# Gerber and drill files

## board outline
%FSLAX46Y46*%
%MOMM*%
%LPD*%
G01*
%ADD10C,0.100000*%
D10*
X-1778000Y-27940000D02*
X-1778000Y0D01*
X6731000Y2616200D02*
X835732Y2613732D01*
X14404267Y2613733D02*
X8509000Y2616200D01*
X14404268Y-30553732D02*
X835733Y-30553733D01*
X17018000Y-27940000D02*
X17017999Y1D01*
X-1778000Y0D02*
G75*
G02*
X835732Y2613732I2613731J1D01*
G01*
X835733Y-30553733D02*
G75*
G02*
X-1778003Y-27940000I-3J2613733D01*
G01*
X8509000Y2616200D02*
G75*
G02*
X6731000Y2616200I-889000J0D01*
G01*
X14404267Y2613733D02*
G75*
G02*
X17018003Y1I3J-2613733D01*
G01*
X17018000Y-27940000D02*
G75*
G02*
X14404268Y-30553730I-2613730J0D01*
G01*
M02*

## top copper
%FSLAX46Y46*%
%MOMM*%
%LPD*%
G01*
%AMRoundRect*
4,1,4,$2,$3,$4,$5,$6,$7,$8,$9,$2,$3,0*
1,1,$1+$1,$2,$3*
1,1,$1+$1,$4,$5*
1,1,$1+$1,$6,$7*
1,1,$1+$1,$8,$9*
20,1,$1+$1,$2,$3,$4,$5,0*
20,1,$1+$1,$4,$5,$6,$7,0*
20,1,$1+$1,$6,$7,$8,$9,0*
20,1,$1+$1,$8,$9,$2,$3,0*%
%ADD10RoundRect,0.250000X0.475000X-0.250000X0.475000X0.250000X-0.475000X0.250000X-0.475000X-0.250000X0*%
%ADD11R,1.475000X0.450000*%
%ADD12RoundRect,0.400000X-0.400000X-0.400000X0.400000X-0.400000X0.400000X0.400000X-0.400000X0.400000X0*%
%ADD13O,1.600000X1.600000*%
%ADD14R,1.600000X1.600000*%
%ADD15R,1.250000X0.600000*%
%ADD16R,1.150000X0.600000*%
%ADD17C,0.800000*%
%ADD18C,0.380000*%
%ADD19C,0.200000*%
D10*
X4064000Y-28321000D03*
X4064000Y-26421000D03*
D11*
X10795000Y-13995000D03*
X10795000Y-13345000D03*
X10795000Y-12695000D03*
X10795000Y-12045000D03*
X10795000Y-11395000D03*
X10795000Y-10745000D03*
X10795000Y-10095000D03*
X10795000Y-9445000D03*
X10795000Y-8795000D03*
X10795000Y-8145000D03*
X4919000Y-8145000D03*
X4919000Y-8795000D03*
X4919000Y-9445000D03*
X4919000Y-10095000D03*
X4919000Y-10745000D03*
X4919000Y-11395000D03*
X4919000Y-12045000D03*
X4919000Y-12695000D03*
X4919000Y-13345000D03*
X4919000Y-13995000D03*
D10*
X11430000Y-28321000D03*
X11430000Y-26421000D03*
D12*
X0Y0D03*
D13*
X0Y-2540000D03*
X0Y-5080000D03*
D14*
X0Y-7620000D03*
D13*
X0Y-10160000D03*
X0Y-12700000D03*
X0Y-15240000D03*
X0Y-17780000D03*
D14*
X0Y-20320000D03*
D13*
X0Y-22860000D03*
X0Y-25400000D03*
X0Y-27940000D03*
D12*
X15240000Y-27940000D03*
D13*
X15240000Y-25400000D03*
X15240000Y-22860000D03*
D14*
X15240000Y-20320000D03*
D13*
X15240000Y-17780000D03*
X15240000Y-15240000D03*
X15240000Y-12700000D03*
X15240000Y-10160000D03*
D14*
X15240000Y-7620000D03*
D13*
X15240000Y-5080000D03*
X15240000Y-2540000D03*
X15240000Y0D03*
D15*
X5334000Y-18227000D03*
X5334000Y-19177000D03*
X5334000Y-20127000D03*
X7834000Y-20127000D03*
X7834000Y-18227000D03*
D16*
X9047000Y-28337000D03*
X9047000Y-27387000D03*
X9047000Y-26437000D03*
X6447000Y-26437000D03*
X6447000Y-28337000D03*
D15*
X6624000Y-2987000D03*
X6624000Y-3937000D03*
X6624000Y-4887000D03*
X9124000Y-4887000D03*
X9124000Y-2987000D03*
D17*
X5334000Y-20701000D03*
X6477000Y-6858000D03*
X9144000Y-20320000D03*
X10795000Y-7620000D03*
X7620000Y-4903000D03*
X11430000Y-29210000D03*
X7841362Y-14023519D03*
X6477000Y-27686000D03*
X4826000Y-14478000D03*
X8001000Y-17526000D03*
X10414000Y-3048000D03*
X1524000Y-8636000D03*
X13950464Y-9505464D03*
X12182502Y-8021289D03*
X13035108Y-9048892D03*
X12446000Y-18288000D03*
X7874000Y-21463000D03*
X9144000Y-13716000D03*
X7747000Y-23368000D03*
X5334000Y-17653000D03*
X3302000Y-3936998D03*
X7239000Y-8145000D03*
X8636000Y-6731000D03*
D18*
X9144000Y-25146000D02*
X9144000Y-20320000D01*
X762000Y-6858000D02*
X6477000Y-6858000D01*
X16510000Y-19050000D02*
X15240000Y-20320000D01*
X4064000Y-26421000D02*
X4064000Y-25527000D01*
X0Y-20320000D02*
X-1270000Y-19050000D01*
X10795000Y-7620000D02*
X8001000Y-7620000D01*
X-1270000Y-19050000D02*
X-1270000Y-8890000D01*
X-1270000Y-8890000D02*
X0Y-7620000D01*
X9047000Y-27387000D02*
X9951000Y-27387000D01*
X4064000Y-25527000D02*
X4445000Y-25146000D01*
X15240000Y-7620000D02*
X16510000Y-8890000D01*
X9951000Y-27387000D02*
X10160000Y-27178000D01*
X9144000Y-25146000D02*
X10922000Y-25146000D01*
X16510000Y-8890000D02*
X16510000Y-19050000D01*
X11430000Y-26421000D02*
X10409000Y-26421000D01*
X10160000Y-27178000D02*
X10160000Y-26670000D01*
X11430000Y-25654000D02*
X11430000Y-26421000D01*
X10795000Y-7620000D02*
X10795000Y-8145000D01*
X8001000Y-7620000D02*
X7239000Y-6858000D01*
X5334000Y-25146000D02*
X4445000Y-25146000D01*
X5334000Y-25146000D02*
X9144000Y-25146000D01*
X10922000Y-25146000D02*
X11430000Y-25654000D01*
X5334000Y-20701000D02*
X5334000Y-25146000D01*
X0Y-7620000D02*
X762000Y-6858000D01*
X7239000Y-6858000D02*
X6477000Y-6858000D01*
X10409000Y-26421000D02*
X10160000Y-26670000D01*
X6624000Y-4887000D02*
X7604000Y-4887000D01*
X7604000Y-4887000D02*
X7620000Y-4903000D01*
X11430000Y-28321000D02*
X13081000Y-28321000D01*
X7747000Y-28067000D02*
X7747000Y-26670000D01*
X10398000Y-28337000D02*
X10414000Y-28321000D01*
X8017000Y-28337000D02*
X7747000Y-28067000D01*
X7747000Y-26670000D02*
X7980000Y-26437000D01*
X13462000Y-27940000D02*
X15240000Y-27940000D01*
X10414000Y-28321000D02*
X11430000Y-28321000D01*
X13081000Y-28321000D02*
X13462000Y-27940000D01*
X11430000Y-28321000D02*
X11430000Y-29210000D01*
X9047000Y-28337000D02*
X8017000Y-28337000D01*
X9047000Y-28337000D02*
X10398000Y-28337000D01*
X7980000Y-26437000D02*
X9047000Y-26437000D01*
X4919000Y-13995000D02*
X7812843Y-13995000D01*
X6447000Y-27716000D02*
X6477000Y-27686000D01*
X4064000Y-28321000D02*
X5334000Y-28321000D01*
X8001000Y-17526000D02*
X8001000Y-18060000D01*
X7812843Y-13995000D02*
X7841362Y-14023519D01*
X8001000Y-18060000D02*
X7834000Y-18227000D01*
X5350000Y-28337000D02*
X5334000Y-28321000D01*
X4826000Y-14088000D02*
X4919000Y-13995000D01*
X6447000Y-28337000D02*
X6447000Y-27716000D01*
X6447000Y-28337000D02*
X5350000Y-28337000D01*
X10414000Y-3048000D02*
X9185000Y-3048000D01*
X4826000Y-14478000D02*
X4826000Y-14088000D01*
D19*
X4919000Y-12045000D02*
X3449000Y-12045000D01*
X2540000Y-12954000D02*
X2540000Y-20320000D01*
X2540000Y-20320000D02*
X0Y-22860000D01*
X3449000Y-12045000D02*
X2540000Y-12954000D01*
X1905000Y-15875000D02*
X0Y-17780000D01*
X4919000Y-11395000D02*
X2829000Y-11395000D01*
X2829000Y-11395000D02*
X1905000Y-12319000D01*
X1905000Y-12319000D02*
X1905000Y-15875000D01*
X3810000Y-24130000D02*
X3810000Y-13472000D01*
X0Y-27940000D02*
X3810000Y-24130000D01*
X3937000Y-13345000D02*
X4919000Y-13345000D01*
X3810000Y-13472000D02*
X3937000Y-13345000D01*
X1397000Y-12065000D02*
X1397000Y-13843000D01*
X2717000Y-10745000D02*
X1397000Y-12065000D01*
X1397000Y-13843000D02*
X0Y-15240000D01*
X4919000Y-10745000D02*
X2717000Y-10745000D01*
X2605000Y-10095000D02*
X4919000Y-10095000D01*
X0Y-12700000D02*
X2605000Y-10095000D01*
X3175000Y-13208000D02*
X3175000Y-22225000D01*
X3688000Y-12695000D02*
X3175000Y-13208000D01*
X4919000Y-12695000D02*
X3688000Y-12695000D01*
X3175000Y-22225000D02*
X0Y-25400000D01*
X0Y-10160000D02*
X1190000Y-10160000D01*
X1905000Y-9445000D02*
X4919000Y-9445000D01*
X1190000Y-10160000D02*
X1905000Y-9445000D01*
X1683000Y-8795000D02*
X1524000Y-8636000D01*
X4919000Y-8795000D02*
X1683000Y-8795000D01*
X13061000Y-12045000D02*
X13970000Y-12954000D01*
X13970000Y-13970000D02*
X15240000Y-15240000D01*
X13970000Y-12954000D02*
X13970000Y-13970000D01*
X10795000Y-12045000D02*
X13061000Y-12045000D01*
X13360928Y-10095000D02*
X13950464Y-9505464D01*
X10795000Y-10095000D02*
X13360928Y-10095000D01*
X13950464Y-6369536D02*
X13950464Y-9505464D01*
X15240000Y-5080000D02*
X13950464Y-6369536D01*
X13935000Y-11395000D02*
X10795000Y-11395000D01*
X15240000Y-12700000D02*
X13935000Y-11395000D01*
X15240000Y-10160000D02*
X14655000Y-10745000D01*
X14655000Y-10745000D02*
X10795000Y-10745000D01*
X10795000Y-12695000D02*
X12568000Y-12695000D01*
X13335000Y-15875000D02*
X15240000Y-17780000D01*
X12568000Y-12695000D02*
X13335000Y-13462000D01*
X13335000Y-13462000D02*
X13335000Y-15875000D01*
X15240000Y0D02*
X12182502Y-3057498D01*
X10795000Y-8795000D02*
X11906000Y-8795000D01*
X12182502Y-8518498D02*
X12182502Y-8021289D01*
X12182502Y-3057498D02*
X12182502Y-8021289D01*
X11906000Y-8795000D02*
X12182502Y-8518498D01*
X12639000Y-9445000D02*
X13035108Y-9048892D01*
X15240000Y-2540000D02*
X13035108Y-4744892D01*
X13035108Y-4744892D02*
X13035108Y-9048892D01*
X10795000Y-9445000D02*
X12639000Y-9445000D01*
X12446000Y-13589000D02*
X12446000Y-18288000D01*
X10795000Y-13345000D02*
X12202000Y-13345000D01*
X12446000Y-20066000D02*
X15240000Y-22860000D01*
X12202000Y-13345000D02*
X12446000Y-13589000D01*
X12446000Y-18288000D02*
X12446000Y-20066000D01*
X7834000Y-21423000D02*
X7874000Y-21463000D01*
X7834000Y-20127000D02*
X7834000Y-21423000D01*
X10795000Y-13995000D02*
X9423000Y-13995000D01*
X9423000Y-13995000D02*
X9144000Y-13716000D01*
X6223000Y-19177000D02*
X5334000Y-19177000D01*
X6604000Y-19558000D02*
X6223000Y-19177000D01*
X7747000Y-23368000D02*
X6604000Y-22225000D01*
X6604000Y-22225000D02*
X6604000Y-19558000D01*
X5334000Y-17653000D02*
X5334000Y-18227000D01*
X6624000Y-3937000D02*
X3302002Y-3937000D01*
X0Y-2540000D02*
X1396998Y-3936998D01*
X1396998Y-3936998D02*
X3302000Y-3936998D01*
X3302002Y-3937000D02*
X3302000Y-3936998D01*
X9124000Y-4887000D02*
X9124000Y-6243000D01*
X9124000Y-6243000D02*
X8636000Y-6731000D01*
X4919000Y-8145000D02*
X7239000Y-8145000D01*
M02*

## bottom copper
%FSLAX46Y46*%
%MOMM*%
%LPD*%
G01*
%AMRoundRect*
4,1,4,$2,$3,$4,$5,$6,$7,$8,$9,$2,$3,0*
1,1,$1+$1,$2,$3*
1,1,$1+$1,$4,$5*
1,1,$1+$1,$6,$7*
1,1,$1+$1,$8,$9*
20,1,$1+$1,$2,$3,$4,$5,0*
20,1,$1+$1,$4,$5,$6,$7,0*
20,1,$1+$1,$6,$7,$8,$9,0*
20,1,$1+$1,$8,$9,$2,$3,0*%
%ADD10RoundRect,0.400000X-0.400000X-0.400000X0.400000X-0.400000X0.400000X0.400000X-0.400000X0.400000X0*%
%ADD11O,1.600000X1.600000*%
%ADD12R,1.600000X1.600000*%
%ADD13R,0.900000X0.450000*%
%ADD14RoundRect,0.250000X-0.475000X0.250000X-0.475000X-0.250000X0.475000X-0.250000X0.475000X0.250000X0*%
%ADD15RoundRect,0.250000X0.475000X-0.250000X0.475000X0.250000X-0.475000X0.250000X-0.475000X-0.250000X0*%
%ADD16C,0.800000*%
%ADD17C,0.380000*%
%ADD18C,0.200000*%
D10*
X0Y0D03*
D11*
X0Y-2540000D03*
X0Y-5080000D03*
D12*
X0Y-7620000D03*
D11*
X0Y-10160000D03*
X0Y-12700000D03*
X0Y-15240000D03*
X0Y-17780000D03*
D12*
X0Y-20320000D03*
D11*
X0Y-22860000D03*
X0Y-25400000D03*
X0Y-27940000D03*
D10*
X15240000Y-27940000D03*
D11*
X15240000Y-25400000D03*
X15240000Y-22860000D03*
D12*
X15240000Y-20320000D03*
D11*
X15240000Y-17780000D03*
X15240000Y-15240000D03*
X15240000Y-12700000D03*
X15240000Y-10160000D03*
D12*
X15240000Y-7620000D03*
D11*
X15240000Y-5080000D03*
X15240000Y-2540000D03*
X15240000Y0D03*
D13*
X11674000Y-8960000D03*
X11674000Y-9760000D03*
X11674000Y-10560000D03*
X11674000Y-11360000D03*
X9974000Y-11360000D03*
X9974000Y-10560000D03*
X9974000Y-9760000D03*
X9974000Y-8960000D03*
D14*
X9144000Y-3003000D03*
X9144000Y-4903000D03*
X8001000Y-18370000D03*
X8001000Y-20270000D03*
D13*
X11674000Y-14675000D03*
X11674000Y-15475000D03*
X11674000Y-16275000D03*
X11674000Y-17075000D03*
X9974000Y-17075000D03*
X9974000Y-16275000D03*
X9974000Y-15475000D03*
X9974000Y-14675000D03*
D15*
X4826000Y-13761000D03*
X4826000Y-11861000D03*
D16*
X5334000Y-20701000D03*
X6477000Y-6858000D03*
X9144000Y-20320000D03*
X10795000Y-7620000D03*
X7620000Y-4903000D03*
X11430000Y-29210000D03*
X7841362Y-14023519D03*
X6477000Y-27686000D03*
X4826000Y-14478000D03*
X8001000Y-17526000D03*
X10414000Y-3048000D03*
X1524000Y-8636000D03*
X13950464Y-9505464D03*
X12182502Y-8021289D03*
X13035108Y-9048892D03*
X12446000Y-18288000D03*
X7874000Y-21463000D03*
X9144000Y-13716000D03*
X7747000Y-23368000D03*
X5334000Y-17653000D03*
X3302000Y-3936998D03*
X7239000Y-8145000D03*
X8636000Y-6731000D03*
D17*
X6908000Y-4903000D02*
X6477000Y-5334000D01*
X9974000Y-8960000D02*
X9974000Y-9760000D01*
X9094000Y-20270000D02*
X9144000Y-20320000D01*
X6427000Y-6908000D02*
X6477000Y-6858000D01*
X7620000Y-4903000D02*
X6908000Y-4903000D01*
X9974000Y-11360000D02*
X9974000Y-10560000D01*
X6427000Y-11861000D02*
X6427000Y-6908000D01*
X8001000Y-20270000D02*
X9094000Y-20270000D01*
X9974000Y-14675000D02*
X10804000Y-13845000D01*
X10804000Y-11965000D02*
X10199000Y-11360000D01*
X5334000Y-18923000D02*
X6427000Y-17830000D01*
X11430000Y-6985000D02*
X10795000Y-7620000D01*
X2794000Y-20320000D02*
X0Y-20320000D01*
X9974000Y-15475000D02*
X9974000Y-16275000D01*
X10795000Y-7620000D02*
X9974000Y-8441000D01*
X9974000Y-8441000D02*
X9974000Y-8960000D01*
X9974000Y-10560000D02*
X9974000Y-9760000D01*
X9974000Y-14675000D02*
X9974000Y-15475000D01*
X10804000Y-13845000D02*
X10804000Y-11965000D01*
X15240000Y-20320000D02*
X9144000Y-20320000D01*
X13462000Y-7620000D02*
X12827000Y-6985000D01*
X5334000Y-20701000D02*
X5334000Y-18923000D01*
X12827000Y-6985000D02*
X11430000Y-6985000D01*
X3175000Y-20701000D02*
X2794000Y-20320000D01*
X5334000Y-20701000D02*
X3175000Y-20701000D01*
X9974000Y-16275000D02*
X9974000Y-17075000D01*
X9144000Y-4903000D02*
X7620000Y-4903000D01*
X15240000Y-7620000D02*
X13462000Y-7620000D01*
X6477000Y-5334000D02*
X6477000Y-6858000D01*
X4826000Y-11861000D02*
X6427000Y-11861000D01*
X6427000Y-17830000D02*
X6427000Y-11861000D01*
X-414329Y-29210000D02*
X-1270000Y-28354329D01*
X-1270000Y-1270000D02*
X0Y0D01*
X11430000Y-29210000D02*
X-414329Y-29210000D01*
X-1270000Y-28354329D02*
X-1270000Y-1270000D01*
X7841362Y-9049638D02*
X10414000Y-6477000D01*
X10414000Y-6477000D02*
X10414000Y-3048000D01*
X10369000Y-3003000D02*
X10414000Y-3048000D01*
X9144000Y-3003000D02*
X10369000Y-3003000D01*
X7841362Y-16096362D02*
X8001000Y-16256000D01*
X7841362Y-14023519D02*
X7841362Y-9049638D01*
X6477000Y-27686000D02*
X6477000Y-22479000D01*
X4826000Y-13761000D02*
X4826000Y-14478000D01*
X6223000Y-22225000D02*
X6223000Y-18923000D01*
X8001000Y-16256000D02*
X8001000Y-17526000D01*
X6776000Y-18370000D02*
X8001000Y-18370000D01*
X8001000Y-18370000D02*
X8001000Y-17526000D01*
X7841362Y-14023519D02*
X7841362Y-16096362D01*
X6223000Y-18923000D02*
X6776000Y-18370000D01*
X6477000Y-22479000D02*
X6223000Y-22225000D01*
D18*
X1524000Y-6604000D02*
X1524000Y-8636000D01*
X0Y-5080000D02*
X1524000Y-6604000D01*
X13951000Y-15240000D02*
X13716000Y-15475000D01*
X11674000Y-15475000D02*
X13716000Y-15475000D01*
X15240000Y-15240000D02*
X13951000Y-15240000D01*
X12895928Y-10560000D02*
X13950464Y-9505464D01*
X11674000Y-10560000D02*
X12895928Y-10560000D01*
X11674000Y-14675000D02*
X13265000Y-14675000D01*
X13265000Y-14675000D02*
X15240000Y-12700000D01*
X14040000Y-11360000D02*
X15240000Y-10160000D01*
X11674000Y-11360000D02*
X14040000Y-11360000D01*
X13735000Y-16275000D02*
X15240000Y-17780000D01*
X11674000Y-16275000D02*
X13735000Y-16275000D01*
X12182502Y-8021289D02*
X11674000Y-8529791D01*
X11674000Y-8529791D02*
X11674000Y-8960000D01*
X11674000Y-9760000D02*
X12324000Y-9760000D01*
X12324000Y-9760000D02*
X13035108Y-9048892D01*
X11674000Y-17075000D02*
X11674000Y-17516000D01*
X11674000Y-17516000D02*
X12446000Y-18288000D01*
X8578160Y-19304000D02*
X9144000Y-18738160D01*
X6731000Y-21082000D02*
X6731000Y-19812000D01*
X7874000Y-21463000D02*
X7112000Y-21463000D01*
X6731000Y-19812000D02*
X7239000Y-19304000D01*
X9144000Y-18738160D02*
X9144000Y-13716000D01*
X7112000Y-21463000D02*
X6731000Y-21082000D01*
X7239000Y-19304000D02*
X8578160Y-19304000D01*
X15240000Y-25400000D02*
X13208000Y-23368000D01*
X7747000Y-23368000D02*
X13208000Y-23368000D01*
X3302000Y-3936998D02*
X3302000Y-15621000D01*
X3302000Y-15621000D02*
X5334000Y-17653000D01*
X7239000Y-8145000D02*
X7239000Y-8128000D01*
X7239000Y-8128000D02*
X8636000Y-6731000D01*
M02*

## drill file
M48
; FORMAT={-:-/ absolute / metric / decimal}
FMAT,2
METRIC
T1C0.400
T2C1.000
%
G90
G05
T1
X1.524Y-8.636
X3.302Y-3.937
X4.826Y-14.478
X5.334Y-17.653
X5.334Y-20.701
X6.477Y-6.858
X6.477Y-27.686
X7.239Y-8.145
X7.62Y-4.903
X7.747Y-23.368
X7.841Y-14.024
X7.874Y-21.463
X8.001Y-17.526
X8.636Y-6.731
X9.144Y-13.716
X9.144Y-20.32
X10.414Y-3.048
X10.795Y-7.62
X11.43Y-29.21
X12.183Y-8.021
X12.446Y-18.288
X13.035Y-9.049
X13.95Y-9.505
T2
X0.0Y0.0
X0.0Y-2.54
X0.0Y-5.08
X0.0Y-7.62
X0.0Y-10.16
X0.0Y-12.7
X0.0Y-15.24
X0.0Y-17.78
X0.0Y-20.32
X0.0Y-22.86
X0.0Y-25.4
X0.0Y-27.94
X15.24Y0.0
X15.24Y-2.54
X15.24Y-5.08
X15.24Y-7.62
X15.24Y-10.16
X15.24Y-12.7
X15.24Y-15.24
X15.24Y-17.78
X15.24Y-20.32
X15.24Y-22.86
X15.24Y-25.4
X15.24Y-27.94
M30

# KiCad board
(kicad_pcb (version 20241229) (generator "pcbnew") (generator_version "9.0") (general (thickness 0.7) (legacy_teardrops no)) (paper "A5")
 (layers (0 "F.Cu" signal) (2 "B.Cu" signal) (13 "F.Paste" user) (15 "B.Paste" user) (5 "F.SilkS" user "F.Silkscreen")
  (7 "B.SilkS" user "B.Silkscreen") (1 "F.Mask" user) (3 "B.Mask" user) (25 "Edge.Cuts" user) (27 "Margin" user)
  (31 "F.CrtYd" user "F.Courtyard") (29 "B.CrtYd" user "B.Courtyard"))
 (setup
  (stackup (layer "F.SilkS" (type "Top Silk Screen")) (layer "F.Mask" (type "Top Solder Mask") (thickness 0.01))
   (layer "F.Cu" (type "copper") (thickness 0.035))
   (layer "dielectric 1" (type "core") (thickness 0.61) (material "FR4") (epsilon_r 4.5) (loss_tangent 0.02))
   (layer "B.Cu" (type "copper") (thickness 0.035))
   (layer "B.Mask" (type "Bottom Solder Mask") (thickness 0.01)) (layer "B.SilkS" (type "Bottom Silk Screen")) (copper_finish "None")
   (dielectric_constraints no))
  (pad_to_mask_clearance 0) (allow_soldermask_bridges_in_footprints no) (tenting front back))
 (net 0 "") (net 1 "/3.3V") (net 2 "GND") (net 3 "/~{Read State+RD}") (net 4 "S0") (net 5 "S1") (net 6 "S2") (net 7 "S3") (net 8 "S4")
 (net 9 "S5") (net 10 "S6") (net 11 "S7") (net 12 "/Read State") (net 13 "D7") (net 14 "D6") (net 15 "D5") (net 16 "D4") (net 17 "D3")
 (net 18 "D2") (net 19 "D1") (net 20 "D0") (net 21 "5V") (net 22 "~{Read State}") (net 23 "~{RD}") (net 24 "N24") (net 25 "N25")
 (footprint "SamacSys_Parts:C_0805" (layer "F.Cu") (at 4.064 27.387)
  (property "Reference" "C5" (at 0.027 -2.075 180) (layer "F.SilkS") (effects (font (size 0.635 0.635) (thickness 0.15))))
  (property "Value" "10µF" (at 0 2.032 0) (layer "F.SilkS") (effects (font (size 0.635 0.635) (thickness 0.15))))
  (pad "1" smd roundrect (at 0 0.934 90) (size 1 1.45) (layers "F.Cu" "F.Mask" "F.Paste") (roundrect_rratio 0.25) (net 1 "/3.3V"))
  (pad "2" smd roundrect (at 0 -0.966 90) (size 1 1.45) (layers "F.Cu" "F.Mask" "F.Paste") (roundrect_rratio 0.25) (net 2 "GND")))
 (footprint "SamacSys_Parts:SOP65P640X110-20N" (layer "F.Cu") (at 7.857 11.07 180)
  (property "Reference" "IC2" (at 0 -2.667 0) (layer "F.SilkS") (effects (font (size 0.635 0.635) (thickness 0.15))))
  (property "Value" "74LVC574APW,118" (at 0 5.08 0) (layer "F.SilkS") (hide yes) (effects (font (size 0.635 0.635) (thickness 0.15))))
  (pad "1" smd rect (at -2.938 -2.925 270) (size 0.45 1.475) (layers "F.Cu" "F.Mask" "F.Paste") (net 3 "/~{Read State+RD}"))
  (pad "2" smd rect (at -2.938 -2.275 270) (size 0.45 1.475) (layers "F.Cu" "F.Mask" "F.Paste") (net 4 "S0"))
  (pad "3" smd rect (at -2.938 -1.625 270) (size 0.45 1.475) (layers "F.Cu" "F.Mask" "F.Paste") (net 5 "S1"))
  (pad "4" smd rect (at -2.938 -0.975 270) (size 0.45 1.475) (layers "F.Cu" "F.Mask" "F.Paste") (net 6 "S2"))
  (pad "5" smd rect (at -2.938 -0.325 270) (size 0.45 1.475) (layers "F.Cu" "F.Mask" "F.Paste") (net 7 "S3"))
  (pad "6" smd rect (at -2.938 0.325 270) (size 0.45 1.475) (layers "F.Cu" "F.Mask" "F.Paste") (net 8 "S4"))
  (pad "7" smd rect (at -2.938 0.975 270) (size 0.45 1.475) (layers "F.Cu" "F.Mask" "F.Paste") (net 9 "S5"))
  (pad "8" smd rect (at -2.938 1.625 270) (size 0.45 1.475) (layers "F.Cu" "F.Mask" "F.Paste") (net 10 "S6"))
  (pad "9" smd rect (at -2.938 2.275 270) (size 0.45 1.475) (layers "F.Cu" "F.Mask" "F.Paste") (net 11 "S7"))
  (pad "10" smd rect (at -2.938 2.925 270) (size 0.45 1.475) (layers "F.Cu" "F.Mask" "F.Paste") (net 2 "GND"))
  (pad "11" smd rect (at 2.938 2.925 270) (size 0.45 1.475) (layers "F.Cu" "F.Mask" "F.Paste") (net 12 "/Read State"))
  (pad "12" smd rect (at 2.938 2.275 270) (size 0.45 1.475) (layers "F.Cu" "F.Mask" "F.Paste") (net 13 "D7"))
  (pad "13" smd rect (at 2.938 1.625 270) (size 0.45 1.475) (layers "F.Cu" "F.Mask" "F.Paste") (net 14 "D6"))
  (pad "14" smd rect (at 2.938 0.975 270) (size 0.45 1.475) (layers "F.Cu" "F.Mask" "F.Paste") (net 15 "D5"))
  (pad "15" smd rect (at 2.938 0.325 270) (size 0.45 1.475) (layers "F.Cu" "F.Mask" "F.Paste") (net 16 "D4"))
  (pad "16" smd rect (at 2.938 -0.325 270) (size 0.45 1.475) (layers "F.Cu" "F.Mask" "F.Paste") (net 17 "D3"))
  (pad "17" smd rect (at 2.938 -0.975 270) (size 0.45 1.475) (layers "F.Cu" "F.Mask" "F.Paste") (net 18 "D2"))
  (pad "18" smd rect (at 2.938 -1.625 270) (size 0.45 1.475) (layers "F.Cu" "F.Mask" "F.Paste") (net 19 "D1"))
  (pad "19" smd rect (at 2.938 -2.275 270) (size 0.45 1.475) (layers "F.Cu" "F.Mask" "F.Paste") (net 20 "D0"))
  (pad "20" smd rect (at 2.938 -2.925 270) (size 0.45 1.475) (layers "F.Cu" "F.Mask" "F.Paste") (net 1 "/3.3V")))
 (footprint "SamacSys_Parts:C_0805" (layer "F.Cu") (at 11.43 27.387)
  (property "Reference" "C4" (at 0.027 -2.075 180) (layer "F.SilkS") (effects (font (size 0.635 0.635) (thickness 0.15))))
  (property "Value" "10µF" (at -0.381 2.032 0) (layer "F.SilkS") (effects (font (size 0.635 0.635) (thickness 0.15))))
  (pad "1" smd roundrect (at 0 0.934 90) (size 1 1.45) (layers "F.Cu" "F.Mask" "F.Paste") (roundrect_rratio 0.25) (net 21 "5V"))
  (pad "2" smd roundrect (at 0 -0.966 90) (size 1 1.45) (layers "F.Cu" "F.Mask" "F.Paste") (roundrect_rratio 0.25) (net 2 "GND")))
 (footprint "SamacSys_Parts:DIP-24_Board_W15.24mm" (layer "F.Cu") (at 0 0)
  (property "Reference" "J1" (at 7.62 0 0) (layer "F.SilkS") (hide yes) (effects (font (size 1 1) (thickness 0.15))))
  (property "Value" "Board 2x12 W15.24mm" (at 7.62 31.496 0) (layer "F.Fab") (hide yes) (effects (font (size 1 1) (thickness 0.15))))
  (fp_line (start -1.778 27.94) (end -1.778 0) (stroke (width 0.1) (type solid)) (layer "Edge.Cuts"))
  (fp_line (start 6.731 -2.6162) (end 0.835732 -2.613732) (stroke (width 0.1) (type solid)) (layer "Edge.Cuts"))
  (fp_line (start 14.404267 -2.613733) (end 8.509 -2.6162) (stroke (width 0.1) (type solid)) (layer "Edge.Cuts"))
  (fp_line (start 14.404268 30.553732) (end 0.835733 30.553733) (stroke (width 0.1) (type solid)) (layer "Edge.Cuts"))
  (fp_line (start 17.018 27.94) (end 17.017999 -0.000001) (stroke (width 0.1) (type solid)) (layer "Edge.Cuts"))
  (fp_arc (start -1.778 0) (mid -1.012456 -1.848188) (end 0.835732 -2.613732) (stroke (width 0.1) (type solid)) (layer "Edge.Cuts"))
  (fp_arc (start 0.835733 30.553733) (mid -1.012456 29.788189) (end -1.778 27.94) (stroke (width 0.1) (type solid)) (layer "Edge.Cuts"))
  (fp_arc (start 8.509 -2.6162) (mid 7.62 -1.7272) (end 6.731 -2.6162) (stroke (width 0.1) (type default)) (layer "Edge.Cuts"))
  (fp_arc (start 14.404267 -2.613733) (mid 16.252455 -1.848189) (end 17.017999 -0.000001) (stroke (width 0.1) (type solid))
   (layer "Edge.Cuts"))
  (fp_arc (start 17.018 27.94) (mid 16.252455 29.788187) (end 14.404268 30.553732) (stroke (width 0.1) (type solid)) (layer "Edge.Cuts"))
  (pad "1" thru_hole roundrect (at 0 0) (size 1.6 1.6) (drill 1) (layers "*.Cu" "*.Mask") (remove_unused_layers no) (roundrect_rratio 0.25)
   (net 21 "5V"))
  (pad "2" thru_hole oval (at 0 2.54) (size 1.6 1.6) (drill 1) (layers "*.Cu" "*.Mask") (remove_unused_layers no) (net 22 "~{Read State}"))
  (pad "3" thru_hole oval (at 0 5.08) (size 1.6 1.6) (drill 1) (layers "*.Cu" "*.Mask") (remove_unused_layers no) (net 13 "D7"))
  (pad "4" thru_hole rect (at 0 7.62) (size 1.6 1.6) (drill 1) (layers "*.Cu" "*.Mask") (remove_unused_layers no) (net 2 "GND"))
  (pad "5" thru_hole oval (at 0 10.16) (size 1.6 1.6) (drill 1) (layers "*.Cu" "*.Mask") (remove_unused_layers no) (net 14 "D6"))
  (pad "6" thru_hole oval (at 0 12.7) (size 1.6 1.6) (drill 1) (layers "*.Cu" "*.Mask") (remove_unused_layers no) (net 15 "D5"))
  (pad "7" thru_hole oval (at 0 15.24) (size 1.6 1.6) (drill 1) (layers "*.Cu" "*.Mask") (remove_unused_layers no) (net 16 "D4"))
  (pad "8" thru_hole oval (at 0 17.78) (size 1.6 1.6) (drill 1) (layers "*.Cu" "*.Mask") (remove_unused_layers no) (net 17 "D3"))
  (pad "9" thru_hole rect (at 0 20.32) (size 1.6 1.6) (drill 1) (layers "*.Cu" "*.Mask") (remove_unused_layers no) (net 2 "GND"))
  (pad "10" thru_hole oval (at 0 22.86) (size 1.6 1.6) (drill 1) (layers "*.Cu" "*.Mask") (remove_unused_layers no) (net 18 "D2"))
  (pad "11" thru_hole oval (at 0 25.4) (size 1.6 1.6) (drill 1) (layers "*.Cu" "*.Mask") (remove_unused_layers no) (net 19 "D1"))
  (pad "12" thru_hole oval (at 0 27.94) (size 1.6 1.6) (drill 1) (layers "*.Cu" "*.Mask") (remove_unused_layers no) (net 20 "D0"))
  (pad "13" thru_hole roundrect (at 15.24 27.94) (size 1.6 1.6) (drill 1) (layers "*.Cu" "*.Mask") (remove_unused_layers no)
   (roundrect_rratio 0.25) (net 21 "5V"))
  (pad "14" thru_hole oval (at 15.24 25.4) (size 1.6 1.6) (drill 1) (layers "*.Cu" "*.Mask") (remove_unused_layers no) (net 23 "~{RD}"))
  (pad "15" thru_hole oval (at 15.24 22.86) (size 1.6 1.6) (drill 1) (layers "*.Cu" "*.Mask") (remove_unused_layers no) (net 4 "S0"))
  (pad "16" thru_hole rect (at 15.24 20.32) (size 1.6 1.6) (drill 1) (layers "*.Cu" "*.Mask") (remove_unused_layers no) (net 2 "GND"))
  (pad "17" thru_hole oval (at 15.24 17.78 180) (size 1.6 1.6) (drill 1) (layers "*.Cu" "*.Mask") (remove_unused_layers no) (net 5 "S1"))
  (pad "18" thru_hole oval (at 15.24 15.24 180) (size 1.6 1.6) (drill 1) (layers "*.Cu" "*.Mask") (remove_unused_layers no) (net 6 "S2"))
  (pad "19" thru_hole oval (at 15.24 12.7 180) (size 1.6 1.6) (drill 1) (layers "*.Cu" "*.Mask") (remove_unused_layers no) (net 7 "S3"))
  (pad "20" thru_hole oval (at 15.24 10.16 180) (size 1.6 1.6) (drill 1) (layers "*.Cu" "*.Mask") (remove_unused_layers no) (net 8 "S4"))
  (pad "21" thru_hole rect (at 15.24 7.62) (size 1.6 1.6) (drill 1) (layers "*.Cu" "*.Mask") (remove_unused_layers no) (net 2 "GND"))
  (pad "22" thru_hole oval (at 15.24 5.08) (size 1.6 1.6) (drill 1) (layers "*.Cu" "*.Mask") (remove_unused_layers no) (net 9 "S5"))
  (pad "23" thru_hole oval (at 15.24 2.54) (size 1.6 1.6) (drill 1) (layers "*.Cu" "*.Mask") (remove_unused_layers no) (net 10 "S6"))
  (pad "24" thru_hole oval (at 15.24 0) (size 1.6 1.6) (drill 1) (layers "*.Cu" "*.Mask") (remove_unused_layers no) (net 11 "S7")))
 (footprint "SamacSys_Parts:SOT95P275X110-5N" (layer "F.Cu") (at 6.584 19.177)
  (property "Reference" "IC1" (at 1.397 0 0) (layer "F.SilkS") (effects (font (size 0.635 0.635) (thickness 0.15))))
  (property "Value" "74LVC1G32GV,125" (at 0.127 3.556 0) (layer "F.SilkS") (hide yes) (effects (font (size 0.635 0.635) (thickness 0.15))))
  (pad "1" smd rect (at -1.25 -0.95 90) (size 0.6 1.25) (layers "F.Cu" "F.Mask" "F.Paste") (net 22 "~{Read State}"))
  (pad "2" smd rect (at -1.25 0 90) (size 0.6 1.25) (layers "F.Cu" "F.Mask" "F.Paste") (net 23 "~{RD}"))
  (pad "3" smd rect (at -1.25 0.95 90) (size 0.6 1.25) (layers "F.Cu" "F.Mask" "F.Paste") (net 2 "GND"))
  (pad "4" smd rect (at 1.25 0.95 90) (size 0.6 1.25) (layers "F.Cu" "F.Mask" "F.Paste") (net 3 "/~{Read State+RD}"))
  (pad "5" smd rect (at 1.25 -0.95 90) (size 0.6 1.25) (layers "F.Cu" "F.Mask" "F.Paste") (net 1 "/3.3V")))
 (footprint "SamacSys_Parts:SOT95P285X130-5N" (layer "F.Cu") (at 7.747 27.387 180)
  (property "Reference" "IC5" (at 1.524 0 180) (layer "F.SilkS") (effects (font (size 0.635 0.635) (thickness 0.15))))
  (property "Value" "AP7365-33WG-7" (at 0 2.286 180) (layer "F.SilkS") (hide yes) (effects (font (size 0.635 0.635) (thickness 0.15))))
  (pad "1" smd rect (at -1.3 -0.95 270) (size 0.6 1.15) (layers "F.Cu" "F.Mask" "F.Paste") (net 21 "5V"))
  (pad "2" smd rect (at -1.3 0 270) (size 0.6 1.15) (layers "F.Cu" "F.Mask" "F.Paste") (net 2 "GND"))
  (pad "3" smd rect (at -1.3 0.95 270) (size 0.6 1.15) (layers "F.Cu" "F.Mask" "F.Paste") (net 21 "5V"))
  (pad "4" smd rect (at 1.3 0.95 270) (size 0.6 1.15) (layers "F.Cu" "F.Mask" "F.Paste") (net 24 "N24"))
  (pad "5" smd rect (at 1.3 -0.95 270) (size 0.6 1.15) (layers "F.Cu" "F.Mask" "F.Paste") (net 1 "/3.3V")))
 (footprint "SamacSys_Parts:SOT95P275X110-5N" (layer "F.Cu") (at 7.874 3.937)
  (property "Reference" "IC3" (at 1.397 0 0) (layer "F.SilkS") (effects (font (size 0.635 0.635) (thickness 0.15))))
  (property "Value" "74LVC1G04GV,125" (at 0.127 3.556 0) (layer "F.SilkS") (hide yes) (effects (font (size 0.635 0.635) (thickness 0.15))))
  (pad "1" smd rect (at -1.25 -0.95 90) (size 0.6 1.25) (layers "F.Cu" "F.Mask" "F.Paste") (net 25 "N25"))
  (pad "2" smd rect (at -1.25 0 90) (size 0.6 1.25) (layers "F.Cu" "F.Mask" "F.Paste") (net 22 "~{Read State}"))
  (pad "3" smd rect (at -1.25 0.95 90) (size 0.6 1.25) (layers "F.Cu" "F.Mask" "F.Paste") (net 2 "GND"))
  (pad "4" smd rect (at 1.25 0.95 90) (size 0.6 1.25) (layers "F.Cu" "F.Mask" "F.Paste") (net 12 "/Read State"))
  (pad "5" smd rect (at 1.25 -0.95 90) (size 0.6 1.25) (layers "F.Cu" "F.Mask" "F.Paste") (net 1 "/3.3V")))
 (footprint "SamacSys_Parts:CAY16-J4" (layer "B.Cu") (at 10.795 10.16)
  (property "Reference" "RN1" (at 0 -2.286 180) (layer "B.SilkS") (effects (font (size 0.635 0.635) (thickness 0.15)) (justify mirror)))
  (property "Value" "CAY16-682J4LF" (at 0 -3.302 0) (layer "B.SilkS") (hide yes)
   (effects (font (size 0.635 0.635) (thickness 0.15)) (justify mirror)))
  (pad "1" smd rect (at 0.879 -1.2 270) (size 0.45 0.9) (layers "B.Cu" "B.Mask" "B.Paste") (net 11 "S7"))
  (pad "2" smd rect (at 0.879 -0.4 270) (size 0.45 0.9) (layers "B.Cu" "B.Mask" "B.Paste") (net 10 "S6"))
  (pad "3" smd rect (at 0.879 0.4 270) (size 0.45 0.9) (layers "B.Cu" "B.Mask" "B.Paste") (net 9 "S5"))
  (pad "4" smd rect (at 0.879 1.2 270) (size 0.45 0.9) (layers "B.Cu" "B.Mask" "B.Paste") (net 8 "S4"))
  (pad "5" smd rect (at -0.821 1.2 270) (size 0.45 0.9) (layers "B.Cu" "B.Mask" "B.Paste") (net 2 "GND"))
  (pad "6" smd rect (at -0.821 0.4 270) (size 0.45 0.9) (layers "B.Cu" "B.Mask" "B.Paste") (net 2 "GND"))
  (pad "7" smd rect (at -0.821 -0.4 270) (size 0.45 0.9) (layers "B.Cu" "B.Mask" "B.Paste") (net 2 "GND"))
  (pad "8" smd rect (at -0.821 -1.2 270) (size 0.45 0.9) (layers "B.Cu" "B.Mask" "B.Paste") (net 2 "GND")))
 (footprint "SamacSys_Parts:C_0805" (layer "B.Cu") (at 9.144 3.937)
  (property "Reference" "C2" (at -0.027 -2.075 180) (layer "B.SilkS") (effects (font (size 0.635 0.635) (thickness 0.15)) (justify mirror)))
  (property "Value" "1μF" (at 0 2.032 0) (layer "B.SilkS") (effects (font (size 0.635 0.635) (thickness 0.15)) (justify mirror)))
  (pad "1" smd roundrect (at 0 -0.934 270) (size 1 1.45) (layers "B.Cu" "B.Mask" "B.Paste") (roundrect_rratio 0.25) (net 1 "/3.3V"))
  (pad "2" smd roundrect (at 0 0.966 270) (size 1 1.45) (layers "B.Cu" "B.Mask" "B.Paste") (roundrect_rratio 0.25) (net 2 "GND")))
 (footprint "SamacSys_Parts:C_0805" (layer "B.Cu") (at 8.001 19.304)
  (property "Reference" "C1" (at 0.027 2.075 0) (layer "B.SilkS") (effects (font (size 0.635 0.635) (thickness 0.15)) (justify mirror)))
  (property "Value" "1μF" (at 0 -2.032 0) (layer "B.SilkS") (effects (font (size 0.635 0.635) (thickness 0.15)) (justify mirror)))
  (pad "1" smd roundrect (at 0 -0.934 270) (size 1 1.45) (layers "B.Cu" "B.Mask" "B.Paste") (roundrect_rratio 0.25) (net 1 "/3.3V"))
  (pad "2" smd roundrect (at 0 0.966 270) (size 1 1.45) (layers "B.Cu" "B.Mask" "B.Paste") (roundrect_rratio 0.25) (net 2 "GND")))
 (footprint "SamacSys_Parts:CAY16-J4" (layer "B.Cu") (at 10.795 15.875)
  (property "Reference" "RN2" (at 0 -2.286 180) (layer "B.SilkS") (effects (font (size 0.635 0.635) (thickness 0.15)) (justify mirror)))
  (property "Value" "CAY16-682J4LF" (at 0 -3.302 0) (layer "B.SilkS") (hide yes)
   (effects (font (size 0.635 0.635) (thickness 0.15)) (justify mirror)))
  (pad "1" smd rect (at 0.879 -1.2 270) (size 0.45 0.9) (layers "B.Cu" "B.Mask" "B.Paste") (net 7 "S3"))
  (pad "2" smd rect (at 0.879 -0.4 270) (size 0.45 0.9) (layers "B.Cu" "B.Mask" "B.Paste") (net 6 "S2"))
  (pad "3" smd rect (at 0.879 0.4 270) (size 0.45 0.9) (layers "B.Cu" "B.Mask" "B.Paste") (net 5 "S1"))
  (pad "4" smd rect (at 0.879 1.2 270) (size 0.45 0.9) (layers "B.Cu" "B.Mask" "B.Paste") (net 4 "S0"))
  (pad "5" smd rect (at -0.821 1.2 270) (size 0.45 0.9) (layers "B.Cu" "B.Mask" "B.Paste") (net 2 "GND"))
  (pad "6" smd rect (at -0.821 0.4 270) (size 0.45 0.9) (layers "B.Cu" "B.Mask" "B.Paste") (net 2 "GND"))
  (pad "7" smd rect (at -0.821 -0.4 270) (size 0.45 0.9) (layers "B.Cu" "B.Mask" "B.Paste") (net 2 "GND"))
  (pad "8" smd rect (at -0.821 -1.2 270) (size 0.45 0.9) (layers "B.Cu" "B.Mask" "B.Paste") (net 2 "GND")))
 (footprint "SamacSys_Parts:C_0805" (layer "B.Cu") (at 4.826 12.827 180)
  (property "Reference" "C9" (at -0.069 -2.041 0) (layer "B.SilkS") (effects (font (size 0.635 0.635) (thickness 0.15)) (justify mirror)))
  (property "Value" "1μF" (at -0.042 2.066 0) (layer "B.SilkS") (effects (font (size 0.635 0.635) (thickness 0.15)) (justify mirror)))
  (pad "1" smd roundrect (at 0 -0.934 90) (size 1 1.45) (layers "B.Cu" "B.Mask" "B.Paste") (roundrect_rratio 0.25) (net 1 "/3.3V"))
  (pad "2" smd roundrect (at 0 0.966 90) (size 1 1.45) (layers "B.Cu" "B.Mask" "B.Paste") (roundrect_rratio 0.25) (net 2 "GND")))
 (segment (start 9.144 25.146) (end 9.144 20.32) (width 0.38) (layer "F.Cu") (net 2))
 (segment (start 0.762 6.858) (end 6.477 6.858) (width 0.38) (layer "F.Cu") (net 2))
 (segment (start 16.51 19.05) (end 15.24 20.32) (width 0.38) (layer "F.Cu") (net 2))
 (segment (start 4.064 26.421) (end 4.064 25.527) (width 0.38) (layer "F.Cu") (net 2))
 (segment (start 0 20.32) (end -1.27 19.05) (width 0.38) (layer "F.Cu") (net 2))
 (segment (start 10.795 7.62) (end 8.001 7.62) (width 0.38) (layer "F.Cu") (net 2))
 (segment (start -1.27 19.05) (end -1.27 8.89) (width 0.38) (layer "F.Cu") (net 2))
 (segment (start -1.27 8.89) (end 0 7.62) (width 0.38) (layer "F.Cu") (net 2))
 (segment (start 9.047 27.387) (end 9.951 27.387) (width 0.38) (layer "F.Cu") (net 2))
 (segment (start 4.064 25.527) (end 4.445 25.146) (width 0.38) (layer "F.Cu") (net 2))
 (segment (start 15.24 7.62) (end 16.51 8.89) (width 0.38) (layer "F.Cu") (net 2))
 (segment (start 9.951 27.387) (end 10.16 27.178) (width 0.38) (layer "F.Cu") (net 2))
 (segment (start 9.144 25.146) (end 10.922 25.146) (width 0.38) (layer "F.Cu") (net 2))
 (segment (start 16.51 8.89) (end 16.51 19.05) (width 0.38) (layer "F.Cu") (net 2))
 (segment (start 11.43 26.421) (end 10.409 26.421) (width 0.38) (layer "F.Cu") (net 2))
 (segment (start 10.16 27.178) (end 10.16 26.67) (width 0.38) (layer "F.Cu") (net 2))
 (segment (start 11.43 25.654) (end 11.43 26.421) (width 0.38) (layer "F.Cu") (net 2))
 (segment (start 10.795 7.62) (end 10.795 8.145) (width 0.38) (layer "F.Cu") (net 2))
 (segment (start 8.001 7.62) (end 7.239 6.858) (width 0.38) (layer "F.Cu") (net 2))
 (segment (start 5.334 25.146) (end 4.445 25.146) (width 0.38) (layer "F.Cu") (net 2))
 (segment (start 5.334 25.146) (end 9.144 25.146) (width 0.38) (layer "F.Cu") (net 2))
 (segment (start 10.922 25.146) (end 11.43 25.654) (width 0.38) (layer "F.Cu") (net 2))
 (segment (start 5.334 20.701) (end 5.334 25.146) (width 0.38) (layer "F.Cu") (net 2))
 (segment (start 0 7.62) (end 0.762 6.858) (width 0.38) (layer "F.Cu") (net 2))
 (segment (start 7.239 6.858) (end 6.477 6.858) (width 0.38) (layer "F.Cu") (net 2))
 (segment (start 10.409 26.421) (end 10.16 26.67) (width 0.38) (layer "F.Cu") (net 2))
 (segment (start 6.624 4.887) (end 7.604 4.887) (width 0.38) (layer "F.Cu") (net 2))
 (segment (start 7.604 4.887) (end 7.62 4.903) (width 0.38) (layer "F.Cu") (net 2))
 (via (at 5.334 20.701) (size 0.8) (drill 0.4) (layers "F.Cu" "B.Cu") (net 2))
 (via (at 6.477 6.858) (size 0.8) (drill 0.4) (layers "F.Cu" "B.Cu") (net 2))
 (via (at 9.144 20.32) (size 0.8) (drill 0.4) (layers "F.Cu" "B.Cu") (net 2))
 (via (at 10.795 7.62) (size 0.8) (drill 0.4) (layers "F.Cu" "B.Cu") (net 2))
 (via (at 7.62 4.903) (size 0.8) (drill 0.4) (layers "F.Cu" "B.Cu") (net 2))
 (segment (start 6.908 4.903) (end 6.477 5.334) (width 0.38) (layer "B.Cu") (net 2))
 (segment (start 9.974 8.96) (end 9.974 9.76) (width 0.38) (layer "B.Cu") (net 2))
 (segment (start 9.094 20.27) (end 9.144 20.32) (width 0.38) (layer "B.Cu") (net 2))
 (segment (start 6.427 6.908) (end 6.477 6.858) (width 0.38) (layer "B.Cu") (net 2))
 (segment (start 7.62 4.903) (end 6.908 4.903) (width 0.38) (layer "B.Cu") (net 2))
 (segment (start 9.974 11.36) (end 9.974 10.56) (width 0.38) (layer "B.Cu") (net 2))
 (segment (start 6.427 11.861) (end 6.427 6.908) (width 0.38) (layer "B.Cu") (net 2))
 (segment (start 8.001 20.27) (end 9.094 20.27) (width 0.38) (layer "B.Cu") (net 2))
 (segment (start 9.974 14.675) (end 10.804 13.845) (width 0.38) (layer "B.Cu") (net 2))
 (segment (start 10.804 11.965) (end 10.199 11.36) (width 0.38) (layer "B.Cu") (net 2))
 (segment (start 5.334 18.923) (end 6.427 17.83) (width 0.38) (layer "B.Cu") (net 2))
 (segment (start 11.43 6.985) (end 10.795 7.62) (width 0.38) (layer "B.Cu") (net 2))
 (segment (start 2.794 20.32) (end 0 20.32) (width 0.38) (layer "B.Cu") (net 2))
 (segment (start 9.974 15.475) (end 9.974 16.275) (width 0.38) (layer "B.Cu") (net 2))
 (segment (start 10.795 7.62) (end 9.974 8.441) (width 0.38) (layer "B.Cu") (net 2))
 (segment (start 9.974 8.441) (end 9.974 8.96) (width 0.38) (layer "B.Cu") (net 2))
 (segment (start 9.974 10.56) (end 9.974 9.76) (width 0.38) (layer "B.Cu") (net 2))
 (segment (start 9.974 14.675) (end 9.974 15.475) (width 0.38) (layer "B.Cu") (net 2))
 (segment (start 10.804 13.845) (end 10.804 11.965) (width 0.38) (layer "B.Cu") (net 2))
 (segment (start 15.24 20.32) (end 9.144 20.32) (width 0.38) (layer "B.Cu") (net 2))
 (segment (start 13.462 7.62) (end 12.827 6.985) (width 0.38) (layer "B.Cu") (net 2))
 (segment (start 5.334 20.701) (end 5.334 18.923) (width 0.38) (layer "B.Cu") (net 2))
 (segment (start 12.827 6.985) (end 11.43 6.985) (width 0.38) (layer "B.Cu") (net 2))
 (segment (start 3.175 20.701) (end 2.794 20.32) (width 0.38) (layer "B.Cu") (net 2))
 (segment (start 5.334 20.701) (end 3.175 20.701) (width 0.38) (layer "B.Cu") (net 2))
 (segment (start 9.974 16.275) (end 9.974 17.075) (width 0.38) (layer "B.Cu") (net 2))
 (segment (start 9.144 4.903) (end 7.62 4.903) (width 0.38) (layer "B.Cu") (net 2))
 (segment (start 15.24 7.62) (end 13.462 7.62) (width 0.38) (layer "B.Cu") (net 2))
 (segment (start 6.477 5.334) (end 6.477 6.858) (width 0.38) (layer "B.Cu") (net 2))
 (segment (start 4.826 11.861) (end 6.427 11.861) (width 0.38) (layer "B.Cu") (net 2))
 (segment (start 6.427 17.83) (end 6.427 11.861) (width 0.38) (layer "B.Cu") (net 2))
 (segment (start 11.43 28.321) (end 13.081 28.321) (width 0.38) (layer "F.Cu") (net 21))
 (segment (start 7.747 28.067) (end 7.747 26.67) (width 0.38) (layer "F.Cu") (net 21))
 (segment (start 10.398 28.337) (end 10.414 28.321) (width 0.38) (layer "F.Cu") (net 21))
 (segment (start 8.017 28.337) (end 7.747 28.067) (width 0.38) (layer "F.Cu") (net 21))
 (segment (start 7.747 26.67) (end 7.98 26.437) (width 0.38) (layer "F.Cu") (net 21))
 (segment (start 13.462 27.94) (end 15.24 27.94) (width 0.38) (layer "F.Cu") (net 21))
 (segment (start 10.414 28.321) (end 11.43 28.321) (width 0.38) (layer "F.Cu") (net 21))
 (segment (start 13.081 28.321) (end 13.462 27.94) (width 0.38) (layer "F.Cu") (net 21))
 (segment (start 11.43 28.321) (end 11.43 29.21) (width 0.38) (layer "F.Cu") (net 21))
 (segment (start 9.047 28.337) (end 8.017 28.337) (width 0.38) (layer "F.Cu") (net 21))
 (segment (start 9.047 28.337) (end 10.398 28.337) (width 0.38) (layer "F.Cu") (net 21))
 (segment (start 7.98 26.437) (end 9.047 26.437) (width 0.38) (layer "F.Cu") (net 21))
 (via (at 11.43 29.21) (size 0.8) (drill 0.4) (layers "F.Cu" "B.Cu") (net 21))
 (segment (start -0.414329 29.21) (end -1.27 28.354329) (width 0.38) (layer "B.Cu") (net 21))
 (segment (start -1.27 1.27) (end 0 0) (width 0.38) (layer "B.Cu") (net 21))
 (segment (start 11.43 29.21) (end -0.414329 29.21) (width 0.38) (layer "B.Cu") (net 21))
 (segment (start -1.27 28.354329) (end -1.27 1.27) (width 0.38) (layer "B.Cu") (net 21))
 (segment (start 4.919 13.995) (end 7.812843 13.995) (width 0.38) (layer "F.Cu") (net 1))
 (segment (start 6.447 27.716) (end 6.477 27.686) (width 0.38) (layer "F.Cu") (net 1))
 (segment (start 4.064 28.321) (end 5.334 28.321) (width 0.38) (layer "F.Cu") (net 1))
 (segment (start 8.001 17.526) (end 8.001 18.06) (width 0.38) (layer "F.Cu") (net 1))
 (segment (start 7.812843 13.995) (end 7.841362 14.023519) (width 0.38) (layer "F.Cu") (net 1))
 (segment (start 8.001 18.06) (end 7.834 18.227) (width 0.38) (layer "F.Cu") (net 1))
 (segment (start 5.35 28.337) (end 5.334 28.321) (width 0.38) (layer "F.Cu") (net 1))
 (segment (start 4.826 14.088) (end 4.919 13.995) (width 0.38) (layer "F.Cu") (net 1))
 (segment (start 6.447 28.337) (end 6.447 27.716) (width 0.38) (layer "F.Cu") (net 1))
 (segment (start 6.447 28.337) (end 5.35 28.337) (width 0.38) (layer "F.Cu") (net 1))
 (segment (start 10.414 3.048) (end 9.185 3.048) (width 0.38) (layer "F.Cu") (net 1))
 (segment (start 4.826 14.478) (end 4.826 14.088) (width 0.38) (layer "F.Cu") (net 1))
 (via (at 7.841362 14.023519) (size 0.8) (drill 0.4) (layers "F.Cu" "B.Cu") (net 1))
 (via (at 6.477 27.686) (size 0.8) (drill 0.4) (layers "F.Cu" "B.Cu") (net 1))
 (via (at 4.826 14.478) (size 0.8) (drill 0.4) (layers "F.Cu" "B.Cu") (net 1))
 (via (at 8.001 17.526) (size 0.8) (drill 0.4) (layers "F.Cu" "B.Cu") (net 1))
 (via (at 10.414 3.048) (size 0.8) (drill 0.4) (layers "F.Cu" "B.Cu") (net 1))
 (segment (start 7.841362 9.049638) (end 10.414 6.477) (width 0.38) (layer "B.Cu") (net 1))
 (segment (start 10.414 6.477) (end 10.414 3.048) (width 0.38) (layer "B.Cu") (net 1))
 (segment (start 10.369 3.003) (end 10.414 3.048) (width 0.38) (layer "B.Cu") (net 1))
 (segment (start 9.144 3.003) (end 10.369 3.003) (width 0.38) (layer "B.Cu") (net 1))
 (segment (start 7.841362 16.096362) (end 8.001 16.256) (width 0.38) (layer "B.Cu") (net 1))
 (segment (start 7.841362 14.023519) (end 7.841362 9.049638) (width 0.38) (layer "B.Cu") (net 1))
 (segment (start 6.477 27.686) (end 6.477 22.479) (width 0.38) (layer "B.Cu") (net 1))
 (segment (start 4.826 13.761) (end 4.826 14.478) (width 0.38) (layer "B.Cu") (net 1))
 (segment (start 6.223 22.225) (end 6.223 18.923) (width 0.38) (layer "B.Cu") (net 1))
 (segment (start 8.001 16.256) (end 8.001 17.526) (width 0.38) (layer "B.Cu") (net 1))
 (segment (start 6.776 18.37) (end 8.001 18.37) (width 0.38) (layer "B.Cu") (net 1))
 (segment (start 8.001 18.37) (end 8.001 17.526) (width 0.38) (layer "B.Cu") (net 1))
 (segment (start 7.841362 14.023519) (end 7.841362 16.096362) (width 0.38) (layer "B.Cu") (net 1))
 (segment (start 6.223 18.923) (end 6.776 18.37) (width 0.38) (layer "B.Cu") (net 1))
 (segment (start 6.477 22.479) (end 6.223 22.225) (width 0.38) (layer "B.Cu") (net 1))
 (segment (start 4.919 12.045) (end 3.449 12.045) (width 0.2) (layer "F.Cu") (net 18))
 (segment (start 2.54 12.954) (end 2.54 20.32) (width 0.2) (layer "F.Cu") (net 18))
 (segment (start 2.54 20.32) (end 0 22.86) (width 0.2) (layer "F.Cu") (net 18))
 (segment (start 3.449 12.045) (end 2.54 12.954) (width 0.2) (layer "F.Cu") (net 18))
 (segment (start 1.905 15.875) (end 0 17.78) (width 0.2) (layer "F.Cu") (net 17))
 (segment (start 4.919 11.395) (end 2.829 11.395) (width 0.2) (layer "F.Cu") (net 17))
 (segment (start 2.829 11.395) (end 1.905 12.319) (width 0.2) (layer "F.Cu") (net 17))
 (segment (start 1.905 12.319) (end 1.905 15.875) (width 0.2) (layer "F.Cu") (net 17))
 (segment (start 3.81 24.13) (end 3.81 13.472) (width 0.2) (layer "F.Cu") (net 20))
 (segment (start 0 27.94) (end 3.81 24.13) (width 0.2) (layer "F.Cu") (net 20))
 (segment (start 3.937 13.345) (end 4.919 13.345) (width 0.2) (layer "F.Cu") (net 20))
 (segment (start 3.81 13.472) (end 3.937 13.345) (width 0.2) (layer "F.Cu") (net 20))
 (segment (start 1.397 12.065) (end 1.397 13.843) (width 0.2) (layer "F.Cu") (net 16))
 (segment (start 2.717 10.745) (end 1.397 12.065) (width 0.2) (layer "F.Cu") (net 16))
 (segment (start 1.397 13.843) (end 0 15.24) (width 0.2) (layer "F.Cu") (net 16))
 (segment (start 4.919 10.745) (end 2.717 10.745) (width 0.2) (layer "F.Cu") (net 16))
 (segment (start 2.605 10.095) (end 4.919 10.095) (width 0.2) (layer "F.Cu") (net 15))
 (segment (start 0 12.7) (end 2.605 10.095) (width 0.2) (layer "F.Cu") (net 15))
 (segment (start 3.175 13.208) (end 3.175 22.225) (width 0.2) (layer "F.Cu") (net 19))
 (segment (start 3.688 12.695) (end 3.175 13.208) (width 0.2) (layer "F.Cu") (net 19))
 (segment (start 4.919 12.695) (end 3.688 12.695) (width 0.2) (layer "F.Cu") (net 19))
 (segment (start 3.175 22.225) (end 0 25.4) (width 0.2) (layer "F.Cu") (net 19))
 (segment (start 0 10.16) (end 1.19 10.16) (width 0.2) (layer "F.Cu") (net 14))
 (segment (start 1.905 9.445) (end 4.919 9.445) (width 0.2) (layer "F.Cu") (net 14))
 (segment (start 1.19 10.16) (end 1.905 9.445) (width 0.2) (layer "F.Cu") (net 14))
 (segment (start 1.683 8.795) (end 1.524 8.636) (width 0.2) (layer "F.Cu") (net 13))
 (segment (start 4.919 8.795) (end 1.683 8.795) (width 0.2) (layer "F.Cu") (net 13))
 (via (at 1.524 8.636) (size 0.8) (drill 0.4) (layers "F.Cu" "B.Cu") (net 13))
 (segment (start 1.524 6.604) (end 1.524 8.636) (width 0.2) (layer "B.Cu") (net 13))
 (segment (start 0 5.08) (end 1.524 6.604) (width 0.2) (layer "B.Cu") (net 13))
 (segment (start 13.061 12.045) (end 13.97 12.954) (width 0.2) (layer "F.Cu") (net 6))
 (segment (start 13.97 13.97) (end 15.24 15.24) (width 0.2) (layer "F.Cu") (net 6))
 (segment (start 13.97 12.954) (end 13.97 13.97) (width 0.2) (layer "F.Cu") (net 6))
 (segment (start 10.795 12.045) (end 13.061 12.045) (width 0.2) (layer "F.Cu") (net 6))
 (segment (start 13.951 15.24) (end 13.716 15.475) (width 0.2) (layer "B.Cu") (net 6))
 (segment (start 11.674 15.475) (end 13.716 15.475) (width 0.2) (layer "B.Cu") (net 6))
 (segment (start 15.24 15.24) (end 13.951 15.24) (width 0.2) (layer "B.Cu") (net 6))
 (segment (start 13.360928 10.095) (end 13.950464 9.505464) (width 0.2) (layer "F.Cu") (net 9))
 (segment (start 10.795 10.095) (end 13.360928 10.095) (width 0.2) (layer "F.Cu") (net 9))
 (segment (start 13.950464 6.369536) (end 13.950464 9.505464) (width 0.2) (layer "F.Cu") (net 9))
 (segment (start 15.24 5.08) (end 13.950464 6.369536) (width 0.2) (layer "F.Cu") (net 9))
 (via (at 13.950464 9.505464) (size 0.8) (drill 0.4) (layers "F.Cu" "B.Cu") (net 9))
 (segment (start 12.895928 10.56) (end 13.950464 9.505464) (width 0.2) (layer "B.Cu") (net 9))
 (segment (start 11.674 10.56) (end 12.895928 10.56) (width 0.2) (layer "B.Cu") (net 9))
 (segment (start 13.935 11.395) (end 10.795 11.395) (width 0.2) (layer "F.Cu") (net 7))
 (segment (start 15.24 12.7) (end 13.935 11.395) (width 0.2) (layer "F.Cu") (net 7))
 (segment (start 11.674 14.675) (end 13.265 14.675) (width 0.2) (layer "B.Cu") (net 7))
 (segment (start 13.265 14.675) (end 15.24 12.7) (width 0.2) (layer "B.Cu") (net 7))
 (segment (start 15.24 10.16) (end 14.655 10.745) (width 0.2) (layer "F.Cu") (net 8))
 (segment (start 14.655 10.745) (end 10.795 10.745) (width 0.2) (layer "F.Cu") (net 8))
 (segment (start 14.04 11.36) (end 15.24 10.16) (width 0.2) (layer "B.Cu") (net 8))
 (segment (start 11.674 11.36) (end 14.04 11.36) (width 0.2) (layer "B.Cu") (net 8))
 (segment (start 10.795 12.695) (end 12.568 12.695) (width 0.2) (layer "F.Cu") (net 5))
 (segment (start 13.335 15.875) (end 15.24 17.78) (width 0.2) (layer "F.Cu") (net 5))
 (segment (start 12.568 12.695) (end 13.335 13.462) (width 0.2) (layer "F.Cu") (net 5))
 (segment (start 13.335 13.462) (end 13.335 15.875) (width 0.2) (layer "F.Cu") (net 5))
 (segment (start 13.735 16.275) (end 15.24 17.78) (width 0.2) (layer "B.Cu") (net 5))
 (segment (start 11.674 16.275) (end 13.735 16.275) (width 0.2) (layer "B.Cu") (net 5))
 (segment (start 15.24 0) (end 12.182502 3.057498) (width 0.2) (layer "F.Cu") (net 11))
 (segment (start 10.795 8.795) (end 11.906 8.795) (width 0.2) (layer "F.Cu") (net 11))
 (segment (start 12.182502 8.518498) (end 12.182502 8.021289) (width 0.2) (layer "F.Cu") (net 11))
 (segment (start 12.182502 3.057498) (end 12.182502 8.021289) (width 0.2) (layer "F.Cu") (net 11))
 (segment (start 11.906 8.795) (end 12.182502 8.518498) (width 0.2) (layer "F.Cu") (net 11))
 (via (at 12.182502 8.021289) (size 0.8) (drill 0.4) (layers "F.Cu" "B.Cu") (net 11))
 (segment (start 12.182502 8.021289) (end 11.674 8.529791) (width 0.2) (layer "B.Cu") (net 11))
 (segment (start 11.674 8.529791) (end 11.674 8.96) (width 0.2) (layer "B.Cu") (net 11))
 (segment (start 12.639 9.445) (end 13.035108 9.048892) (width 0.2) (layer "F.Cu") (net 10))
 (segment (start 15.24 2.54) (end 13.035108 4.744892) (width 0.2) (layer "F.Cu") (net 10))
 (segment (start 13.035108 4.744892) (end 13.035108 9.048892) (width 0.2) (layer "F.Cu") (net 10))
 (segment (start 10.795 9.445) (end 12.639 9.445) (width 0.2) (layer "F.Cu") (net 10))
 (via (at 13.035108 9.048892) (size 0.8) (drill 0.4) (layers "F.Cu" "B.Cu") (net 10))
 (segment (start 11.674 9.76) (end 12.324 9.76) (width 0.2) (layer "B.Cu") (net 10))
 (segment (start 12.324 9.76) (end 13.035108 9.048892) (width 0.2) (layer "B.Cu") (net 10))
 (segment (start 12.446 13.589) (end 12.446 18.288) (width 0.2) (layer "F.Cu") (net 4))
 (segment (start 10.795 13.345) (end 12.202 13.345) (width 0.2) (layer "F.Cu") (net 4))
 (segment (start 12.446 20.066) (end 15.24 22.86) (width 0.2) (layer "F.Cu") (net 4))
 (segment (start 12.202 13.345) (end 12.446 13.589) (width 0.2) (layer "F.Cu") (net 4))
 (segment (start 12.446 18.288) (end 12.446 20.066) (width 0.2) (layer "F.Cu") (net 4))
 (via (at 12.446 18.288) (size 0.8) (drill 0.4) (layers "F.Cu" "B.Cu") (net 4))
 (segment (start 11.674 17.075) (end 11.674 17.516) (width 0.2) (layer "B.Cu") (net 4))
 (segment (start 11.674 17.516) (end 12.446 18.288) (width 0.2) (layer "B.Cu") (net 4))
 (segment (start 7.834 21.423) (end 7.874 21.463) (width 0.2) (layer "F.Cu") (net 3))
 (segment (start 7.834 20.127) (end 7.834 21.423) (width 0.2) (layer "F.Cu") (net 3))
 (segment (start 10.795 13.995) (end 9.423 13.995) (width 0.2) (layer "F.Cu") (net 3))
 (segment (start 9.423 13.995) (end 9.144 13.716) (width 0.2) (layer "F.Cu") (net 3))
 (via (at 7.874 21.463) (size 0.8) (drill 0.4) (layers "F.Cu" "B.Cu") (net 3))
 (via (at 9.144 13.716) (size 0.8) (drill 0.4) (layers "F.Cu" "B.Cu") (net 3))
 (segment (start 8.57816 19.304) (end 9.144 18.73816) (width 0.2) (layer "B.Cu") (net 3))
 (segment (start 6.731 21.082) (end 6.731 19.812) (width 0.2) (layer "B.Cu") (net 3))
 (segment (start 7.874 21.463) (end 7.112 21.463) (width 0.2) (layer "B.Cu") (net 3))
 (segment (start 6.731 19.812) (end 7.239 19.304) (width 0.2) (layer "B.Cu") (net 3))
 (segment (start 9.144 18.73816) (end 9.144 13.716) (width 0.2) (layer "B.Cu") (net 3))
 (segment (start 7.112 21.463) (end 6.731 21.082) (width 0.2) (layer "B.Cu") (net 3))
 (segment (start 7.239 19.304) (end 8.57816 19.304) (width 0.2) (layer "B.Cu") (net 3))
 (segment (start 6.223 19.177) (end 5.334 19.177) (width 0.2) (layer "F.Cu") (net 23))
 (segment (start 6.604 19.558) (end 6.223 19.177) (width 0.2) (layer "F.Cu") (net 23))
 (segment (start 7.747 23.368) (end 6.604 22.225) (width 0.2) (layer "F.Cu") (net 23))
 (segment (start 6.604 22.225) (end 6.604 19.558) (width 0.2) (layer "F.Cu") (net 23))
 (via (at 7.747 23.368) (size 0.8) (drill 0.4) (layers "F.Cu" "B.Cu") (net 23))
 (segment (start 15.24 25.4) (end 13.208 23.368) (width 0.2) (layer "B.Cu") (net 23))
 (segment (start 7.747 23.368) (end 13.208 23.368) (width 0.2) (layer "B.Cu") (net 23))
 (segment (start 5.334 17.653) (end 5.334 18.227) (width 0.2) (layer "F.Cu") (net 22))
 (segment (start 6.624 3.937) (end 3.302002 3.937) (width 0.2) (layer "F.Cu") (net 22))
 (segment (start 0 2.54) (end 1.396998 3.936998) (width 0.2) (layer "F.Cu") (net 22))
 (segment (start 1.396998 3.936998) (end 3.302 3.936998) (width 0.2) (layer "F.Cu") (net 22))
 (segment (start 3.302002 3.937) (end 3.302 3.936998) (width 0.2) (layer "F.Cu") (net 22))
 (via (at 5.334 17.653) (size 0.8) (drill 0.4) (layers "F.Cu" "B.Cu") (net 22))
 (via (at 3.302 3.936998) (size 0.8) (drill 0.4) (layers "F.Cu" "B.Cu") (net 22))
 (segment (start 3.302 3.936998) (end 3.302 15.621) (width 0.2) (layer "B.Cu") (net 22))
 (segment (start 3.302 15.621) (end 5.334 17.653) (width 0.2) (layer "B.Cu") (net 22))
 (segment (start 9.124 4.887) (end 9.124 6.243) (width 0.2) (layer "F.Cu") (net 12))
 (segment (start 9.124 6.243) (end 8.636 6.731) (width 0.2) (layer "F.Cu") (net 12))
 (segment (start 4.919 8.145) (end 7.239 8.145) (width 0.2) (layer "F.Cu") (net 12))
 (via (at 7.239 8.145) (size 0.8) (drill 0.4) (layers "F.Cu" "B.Cu") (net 12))
 (via (at 8.636 6.731) (size 0.8) (drill 0.4) (layers "F.Cu" "B.Cu") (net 12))
 (segment (start 7.239 8.145) (end 7.239 8.128) (width 0.2) (layer "B.Cu") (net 12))
 (segment (start 7.239 8.128) (end 8.636 6.731) (width 0.2) (layer "B.Cu") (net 12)))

